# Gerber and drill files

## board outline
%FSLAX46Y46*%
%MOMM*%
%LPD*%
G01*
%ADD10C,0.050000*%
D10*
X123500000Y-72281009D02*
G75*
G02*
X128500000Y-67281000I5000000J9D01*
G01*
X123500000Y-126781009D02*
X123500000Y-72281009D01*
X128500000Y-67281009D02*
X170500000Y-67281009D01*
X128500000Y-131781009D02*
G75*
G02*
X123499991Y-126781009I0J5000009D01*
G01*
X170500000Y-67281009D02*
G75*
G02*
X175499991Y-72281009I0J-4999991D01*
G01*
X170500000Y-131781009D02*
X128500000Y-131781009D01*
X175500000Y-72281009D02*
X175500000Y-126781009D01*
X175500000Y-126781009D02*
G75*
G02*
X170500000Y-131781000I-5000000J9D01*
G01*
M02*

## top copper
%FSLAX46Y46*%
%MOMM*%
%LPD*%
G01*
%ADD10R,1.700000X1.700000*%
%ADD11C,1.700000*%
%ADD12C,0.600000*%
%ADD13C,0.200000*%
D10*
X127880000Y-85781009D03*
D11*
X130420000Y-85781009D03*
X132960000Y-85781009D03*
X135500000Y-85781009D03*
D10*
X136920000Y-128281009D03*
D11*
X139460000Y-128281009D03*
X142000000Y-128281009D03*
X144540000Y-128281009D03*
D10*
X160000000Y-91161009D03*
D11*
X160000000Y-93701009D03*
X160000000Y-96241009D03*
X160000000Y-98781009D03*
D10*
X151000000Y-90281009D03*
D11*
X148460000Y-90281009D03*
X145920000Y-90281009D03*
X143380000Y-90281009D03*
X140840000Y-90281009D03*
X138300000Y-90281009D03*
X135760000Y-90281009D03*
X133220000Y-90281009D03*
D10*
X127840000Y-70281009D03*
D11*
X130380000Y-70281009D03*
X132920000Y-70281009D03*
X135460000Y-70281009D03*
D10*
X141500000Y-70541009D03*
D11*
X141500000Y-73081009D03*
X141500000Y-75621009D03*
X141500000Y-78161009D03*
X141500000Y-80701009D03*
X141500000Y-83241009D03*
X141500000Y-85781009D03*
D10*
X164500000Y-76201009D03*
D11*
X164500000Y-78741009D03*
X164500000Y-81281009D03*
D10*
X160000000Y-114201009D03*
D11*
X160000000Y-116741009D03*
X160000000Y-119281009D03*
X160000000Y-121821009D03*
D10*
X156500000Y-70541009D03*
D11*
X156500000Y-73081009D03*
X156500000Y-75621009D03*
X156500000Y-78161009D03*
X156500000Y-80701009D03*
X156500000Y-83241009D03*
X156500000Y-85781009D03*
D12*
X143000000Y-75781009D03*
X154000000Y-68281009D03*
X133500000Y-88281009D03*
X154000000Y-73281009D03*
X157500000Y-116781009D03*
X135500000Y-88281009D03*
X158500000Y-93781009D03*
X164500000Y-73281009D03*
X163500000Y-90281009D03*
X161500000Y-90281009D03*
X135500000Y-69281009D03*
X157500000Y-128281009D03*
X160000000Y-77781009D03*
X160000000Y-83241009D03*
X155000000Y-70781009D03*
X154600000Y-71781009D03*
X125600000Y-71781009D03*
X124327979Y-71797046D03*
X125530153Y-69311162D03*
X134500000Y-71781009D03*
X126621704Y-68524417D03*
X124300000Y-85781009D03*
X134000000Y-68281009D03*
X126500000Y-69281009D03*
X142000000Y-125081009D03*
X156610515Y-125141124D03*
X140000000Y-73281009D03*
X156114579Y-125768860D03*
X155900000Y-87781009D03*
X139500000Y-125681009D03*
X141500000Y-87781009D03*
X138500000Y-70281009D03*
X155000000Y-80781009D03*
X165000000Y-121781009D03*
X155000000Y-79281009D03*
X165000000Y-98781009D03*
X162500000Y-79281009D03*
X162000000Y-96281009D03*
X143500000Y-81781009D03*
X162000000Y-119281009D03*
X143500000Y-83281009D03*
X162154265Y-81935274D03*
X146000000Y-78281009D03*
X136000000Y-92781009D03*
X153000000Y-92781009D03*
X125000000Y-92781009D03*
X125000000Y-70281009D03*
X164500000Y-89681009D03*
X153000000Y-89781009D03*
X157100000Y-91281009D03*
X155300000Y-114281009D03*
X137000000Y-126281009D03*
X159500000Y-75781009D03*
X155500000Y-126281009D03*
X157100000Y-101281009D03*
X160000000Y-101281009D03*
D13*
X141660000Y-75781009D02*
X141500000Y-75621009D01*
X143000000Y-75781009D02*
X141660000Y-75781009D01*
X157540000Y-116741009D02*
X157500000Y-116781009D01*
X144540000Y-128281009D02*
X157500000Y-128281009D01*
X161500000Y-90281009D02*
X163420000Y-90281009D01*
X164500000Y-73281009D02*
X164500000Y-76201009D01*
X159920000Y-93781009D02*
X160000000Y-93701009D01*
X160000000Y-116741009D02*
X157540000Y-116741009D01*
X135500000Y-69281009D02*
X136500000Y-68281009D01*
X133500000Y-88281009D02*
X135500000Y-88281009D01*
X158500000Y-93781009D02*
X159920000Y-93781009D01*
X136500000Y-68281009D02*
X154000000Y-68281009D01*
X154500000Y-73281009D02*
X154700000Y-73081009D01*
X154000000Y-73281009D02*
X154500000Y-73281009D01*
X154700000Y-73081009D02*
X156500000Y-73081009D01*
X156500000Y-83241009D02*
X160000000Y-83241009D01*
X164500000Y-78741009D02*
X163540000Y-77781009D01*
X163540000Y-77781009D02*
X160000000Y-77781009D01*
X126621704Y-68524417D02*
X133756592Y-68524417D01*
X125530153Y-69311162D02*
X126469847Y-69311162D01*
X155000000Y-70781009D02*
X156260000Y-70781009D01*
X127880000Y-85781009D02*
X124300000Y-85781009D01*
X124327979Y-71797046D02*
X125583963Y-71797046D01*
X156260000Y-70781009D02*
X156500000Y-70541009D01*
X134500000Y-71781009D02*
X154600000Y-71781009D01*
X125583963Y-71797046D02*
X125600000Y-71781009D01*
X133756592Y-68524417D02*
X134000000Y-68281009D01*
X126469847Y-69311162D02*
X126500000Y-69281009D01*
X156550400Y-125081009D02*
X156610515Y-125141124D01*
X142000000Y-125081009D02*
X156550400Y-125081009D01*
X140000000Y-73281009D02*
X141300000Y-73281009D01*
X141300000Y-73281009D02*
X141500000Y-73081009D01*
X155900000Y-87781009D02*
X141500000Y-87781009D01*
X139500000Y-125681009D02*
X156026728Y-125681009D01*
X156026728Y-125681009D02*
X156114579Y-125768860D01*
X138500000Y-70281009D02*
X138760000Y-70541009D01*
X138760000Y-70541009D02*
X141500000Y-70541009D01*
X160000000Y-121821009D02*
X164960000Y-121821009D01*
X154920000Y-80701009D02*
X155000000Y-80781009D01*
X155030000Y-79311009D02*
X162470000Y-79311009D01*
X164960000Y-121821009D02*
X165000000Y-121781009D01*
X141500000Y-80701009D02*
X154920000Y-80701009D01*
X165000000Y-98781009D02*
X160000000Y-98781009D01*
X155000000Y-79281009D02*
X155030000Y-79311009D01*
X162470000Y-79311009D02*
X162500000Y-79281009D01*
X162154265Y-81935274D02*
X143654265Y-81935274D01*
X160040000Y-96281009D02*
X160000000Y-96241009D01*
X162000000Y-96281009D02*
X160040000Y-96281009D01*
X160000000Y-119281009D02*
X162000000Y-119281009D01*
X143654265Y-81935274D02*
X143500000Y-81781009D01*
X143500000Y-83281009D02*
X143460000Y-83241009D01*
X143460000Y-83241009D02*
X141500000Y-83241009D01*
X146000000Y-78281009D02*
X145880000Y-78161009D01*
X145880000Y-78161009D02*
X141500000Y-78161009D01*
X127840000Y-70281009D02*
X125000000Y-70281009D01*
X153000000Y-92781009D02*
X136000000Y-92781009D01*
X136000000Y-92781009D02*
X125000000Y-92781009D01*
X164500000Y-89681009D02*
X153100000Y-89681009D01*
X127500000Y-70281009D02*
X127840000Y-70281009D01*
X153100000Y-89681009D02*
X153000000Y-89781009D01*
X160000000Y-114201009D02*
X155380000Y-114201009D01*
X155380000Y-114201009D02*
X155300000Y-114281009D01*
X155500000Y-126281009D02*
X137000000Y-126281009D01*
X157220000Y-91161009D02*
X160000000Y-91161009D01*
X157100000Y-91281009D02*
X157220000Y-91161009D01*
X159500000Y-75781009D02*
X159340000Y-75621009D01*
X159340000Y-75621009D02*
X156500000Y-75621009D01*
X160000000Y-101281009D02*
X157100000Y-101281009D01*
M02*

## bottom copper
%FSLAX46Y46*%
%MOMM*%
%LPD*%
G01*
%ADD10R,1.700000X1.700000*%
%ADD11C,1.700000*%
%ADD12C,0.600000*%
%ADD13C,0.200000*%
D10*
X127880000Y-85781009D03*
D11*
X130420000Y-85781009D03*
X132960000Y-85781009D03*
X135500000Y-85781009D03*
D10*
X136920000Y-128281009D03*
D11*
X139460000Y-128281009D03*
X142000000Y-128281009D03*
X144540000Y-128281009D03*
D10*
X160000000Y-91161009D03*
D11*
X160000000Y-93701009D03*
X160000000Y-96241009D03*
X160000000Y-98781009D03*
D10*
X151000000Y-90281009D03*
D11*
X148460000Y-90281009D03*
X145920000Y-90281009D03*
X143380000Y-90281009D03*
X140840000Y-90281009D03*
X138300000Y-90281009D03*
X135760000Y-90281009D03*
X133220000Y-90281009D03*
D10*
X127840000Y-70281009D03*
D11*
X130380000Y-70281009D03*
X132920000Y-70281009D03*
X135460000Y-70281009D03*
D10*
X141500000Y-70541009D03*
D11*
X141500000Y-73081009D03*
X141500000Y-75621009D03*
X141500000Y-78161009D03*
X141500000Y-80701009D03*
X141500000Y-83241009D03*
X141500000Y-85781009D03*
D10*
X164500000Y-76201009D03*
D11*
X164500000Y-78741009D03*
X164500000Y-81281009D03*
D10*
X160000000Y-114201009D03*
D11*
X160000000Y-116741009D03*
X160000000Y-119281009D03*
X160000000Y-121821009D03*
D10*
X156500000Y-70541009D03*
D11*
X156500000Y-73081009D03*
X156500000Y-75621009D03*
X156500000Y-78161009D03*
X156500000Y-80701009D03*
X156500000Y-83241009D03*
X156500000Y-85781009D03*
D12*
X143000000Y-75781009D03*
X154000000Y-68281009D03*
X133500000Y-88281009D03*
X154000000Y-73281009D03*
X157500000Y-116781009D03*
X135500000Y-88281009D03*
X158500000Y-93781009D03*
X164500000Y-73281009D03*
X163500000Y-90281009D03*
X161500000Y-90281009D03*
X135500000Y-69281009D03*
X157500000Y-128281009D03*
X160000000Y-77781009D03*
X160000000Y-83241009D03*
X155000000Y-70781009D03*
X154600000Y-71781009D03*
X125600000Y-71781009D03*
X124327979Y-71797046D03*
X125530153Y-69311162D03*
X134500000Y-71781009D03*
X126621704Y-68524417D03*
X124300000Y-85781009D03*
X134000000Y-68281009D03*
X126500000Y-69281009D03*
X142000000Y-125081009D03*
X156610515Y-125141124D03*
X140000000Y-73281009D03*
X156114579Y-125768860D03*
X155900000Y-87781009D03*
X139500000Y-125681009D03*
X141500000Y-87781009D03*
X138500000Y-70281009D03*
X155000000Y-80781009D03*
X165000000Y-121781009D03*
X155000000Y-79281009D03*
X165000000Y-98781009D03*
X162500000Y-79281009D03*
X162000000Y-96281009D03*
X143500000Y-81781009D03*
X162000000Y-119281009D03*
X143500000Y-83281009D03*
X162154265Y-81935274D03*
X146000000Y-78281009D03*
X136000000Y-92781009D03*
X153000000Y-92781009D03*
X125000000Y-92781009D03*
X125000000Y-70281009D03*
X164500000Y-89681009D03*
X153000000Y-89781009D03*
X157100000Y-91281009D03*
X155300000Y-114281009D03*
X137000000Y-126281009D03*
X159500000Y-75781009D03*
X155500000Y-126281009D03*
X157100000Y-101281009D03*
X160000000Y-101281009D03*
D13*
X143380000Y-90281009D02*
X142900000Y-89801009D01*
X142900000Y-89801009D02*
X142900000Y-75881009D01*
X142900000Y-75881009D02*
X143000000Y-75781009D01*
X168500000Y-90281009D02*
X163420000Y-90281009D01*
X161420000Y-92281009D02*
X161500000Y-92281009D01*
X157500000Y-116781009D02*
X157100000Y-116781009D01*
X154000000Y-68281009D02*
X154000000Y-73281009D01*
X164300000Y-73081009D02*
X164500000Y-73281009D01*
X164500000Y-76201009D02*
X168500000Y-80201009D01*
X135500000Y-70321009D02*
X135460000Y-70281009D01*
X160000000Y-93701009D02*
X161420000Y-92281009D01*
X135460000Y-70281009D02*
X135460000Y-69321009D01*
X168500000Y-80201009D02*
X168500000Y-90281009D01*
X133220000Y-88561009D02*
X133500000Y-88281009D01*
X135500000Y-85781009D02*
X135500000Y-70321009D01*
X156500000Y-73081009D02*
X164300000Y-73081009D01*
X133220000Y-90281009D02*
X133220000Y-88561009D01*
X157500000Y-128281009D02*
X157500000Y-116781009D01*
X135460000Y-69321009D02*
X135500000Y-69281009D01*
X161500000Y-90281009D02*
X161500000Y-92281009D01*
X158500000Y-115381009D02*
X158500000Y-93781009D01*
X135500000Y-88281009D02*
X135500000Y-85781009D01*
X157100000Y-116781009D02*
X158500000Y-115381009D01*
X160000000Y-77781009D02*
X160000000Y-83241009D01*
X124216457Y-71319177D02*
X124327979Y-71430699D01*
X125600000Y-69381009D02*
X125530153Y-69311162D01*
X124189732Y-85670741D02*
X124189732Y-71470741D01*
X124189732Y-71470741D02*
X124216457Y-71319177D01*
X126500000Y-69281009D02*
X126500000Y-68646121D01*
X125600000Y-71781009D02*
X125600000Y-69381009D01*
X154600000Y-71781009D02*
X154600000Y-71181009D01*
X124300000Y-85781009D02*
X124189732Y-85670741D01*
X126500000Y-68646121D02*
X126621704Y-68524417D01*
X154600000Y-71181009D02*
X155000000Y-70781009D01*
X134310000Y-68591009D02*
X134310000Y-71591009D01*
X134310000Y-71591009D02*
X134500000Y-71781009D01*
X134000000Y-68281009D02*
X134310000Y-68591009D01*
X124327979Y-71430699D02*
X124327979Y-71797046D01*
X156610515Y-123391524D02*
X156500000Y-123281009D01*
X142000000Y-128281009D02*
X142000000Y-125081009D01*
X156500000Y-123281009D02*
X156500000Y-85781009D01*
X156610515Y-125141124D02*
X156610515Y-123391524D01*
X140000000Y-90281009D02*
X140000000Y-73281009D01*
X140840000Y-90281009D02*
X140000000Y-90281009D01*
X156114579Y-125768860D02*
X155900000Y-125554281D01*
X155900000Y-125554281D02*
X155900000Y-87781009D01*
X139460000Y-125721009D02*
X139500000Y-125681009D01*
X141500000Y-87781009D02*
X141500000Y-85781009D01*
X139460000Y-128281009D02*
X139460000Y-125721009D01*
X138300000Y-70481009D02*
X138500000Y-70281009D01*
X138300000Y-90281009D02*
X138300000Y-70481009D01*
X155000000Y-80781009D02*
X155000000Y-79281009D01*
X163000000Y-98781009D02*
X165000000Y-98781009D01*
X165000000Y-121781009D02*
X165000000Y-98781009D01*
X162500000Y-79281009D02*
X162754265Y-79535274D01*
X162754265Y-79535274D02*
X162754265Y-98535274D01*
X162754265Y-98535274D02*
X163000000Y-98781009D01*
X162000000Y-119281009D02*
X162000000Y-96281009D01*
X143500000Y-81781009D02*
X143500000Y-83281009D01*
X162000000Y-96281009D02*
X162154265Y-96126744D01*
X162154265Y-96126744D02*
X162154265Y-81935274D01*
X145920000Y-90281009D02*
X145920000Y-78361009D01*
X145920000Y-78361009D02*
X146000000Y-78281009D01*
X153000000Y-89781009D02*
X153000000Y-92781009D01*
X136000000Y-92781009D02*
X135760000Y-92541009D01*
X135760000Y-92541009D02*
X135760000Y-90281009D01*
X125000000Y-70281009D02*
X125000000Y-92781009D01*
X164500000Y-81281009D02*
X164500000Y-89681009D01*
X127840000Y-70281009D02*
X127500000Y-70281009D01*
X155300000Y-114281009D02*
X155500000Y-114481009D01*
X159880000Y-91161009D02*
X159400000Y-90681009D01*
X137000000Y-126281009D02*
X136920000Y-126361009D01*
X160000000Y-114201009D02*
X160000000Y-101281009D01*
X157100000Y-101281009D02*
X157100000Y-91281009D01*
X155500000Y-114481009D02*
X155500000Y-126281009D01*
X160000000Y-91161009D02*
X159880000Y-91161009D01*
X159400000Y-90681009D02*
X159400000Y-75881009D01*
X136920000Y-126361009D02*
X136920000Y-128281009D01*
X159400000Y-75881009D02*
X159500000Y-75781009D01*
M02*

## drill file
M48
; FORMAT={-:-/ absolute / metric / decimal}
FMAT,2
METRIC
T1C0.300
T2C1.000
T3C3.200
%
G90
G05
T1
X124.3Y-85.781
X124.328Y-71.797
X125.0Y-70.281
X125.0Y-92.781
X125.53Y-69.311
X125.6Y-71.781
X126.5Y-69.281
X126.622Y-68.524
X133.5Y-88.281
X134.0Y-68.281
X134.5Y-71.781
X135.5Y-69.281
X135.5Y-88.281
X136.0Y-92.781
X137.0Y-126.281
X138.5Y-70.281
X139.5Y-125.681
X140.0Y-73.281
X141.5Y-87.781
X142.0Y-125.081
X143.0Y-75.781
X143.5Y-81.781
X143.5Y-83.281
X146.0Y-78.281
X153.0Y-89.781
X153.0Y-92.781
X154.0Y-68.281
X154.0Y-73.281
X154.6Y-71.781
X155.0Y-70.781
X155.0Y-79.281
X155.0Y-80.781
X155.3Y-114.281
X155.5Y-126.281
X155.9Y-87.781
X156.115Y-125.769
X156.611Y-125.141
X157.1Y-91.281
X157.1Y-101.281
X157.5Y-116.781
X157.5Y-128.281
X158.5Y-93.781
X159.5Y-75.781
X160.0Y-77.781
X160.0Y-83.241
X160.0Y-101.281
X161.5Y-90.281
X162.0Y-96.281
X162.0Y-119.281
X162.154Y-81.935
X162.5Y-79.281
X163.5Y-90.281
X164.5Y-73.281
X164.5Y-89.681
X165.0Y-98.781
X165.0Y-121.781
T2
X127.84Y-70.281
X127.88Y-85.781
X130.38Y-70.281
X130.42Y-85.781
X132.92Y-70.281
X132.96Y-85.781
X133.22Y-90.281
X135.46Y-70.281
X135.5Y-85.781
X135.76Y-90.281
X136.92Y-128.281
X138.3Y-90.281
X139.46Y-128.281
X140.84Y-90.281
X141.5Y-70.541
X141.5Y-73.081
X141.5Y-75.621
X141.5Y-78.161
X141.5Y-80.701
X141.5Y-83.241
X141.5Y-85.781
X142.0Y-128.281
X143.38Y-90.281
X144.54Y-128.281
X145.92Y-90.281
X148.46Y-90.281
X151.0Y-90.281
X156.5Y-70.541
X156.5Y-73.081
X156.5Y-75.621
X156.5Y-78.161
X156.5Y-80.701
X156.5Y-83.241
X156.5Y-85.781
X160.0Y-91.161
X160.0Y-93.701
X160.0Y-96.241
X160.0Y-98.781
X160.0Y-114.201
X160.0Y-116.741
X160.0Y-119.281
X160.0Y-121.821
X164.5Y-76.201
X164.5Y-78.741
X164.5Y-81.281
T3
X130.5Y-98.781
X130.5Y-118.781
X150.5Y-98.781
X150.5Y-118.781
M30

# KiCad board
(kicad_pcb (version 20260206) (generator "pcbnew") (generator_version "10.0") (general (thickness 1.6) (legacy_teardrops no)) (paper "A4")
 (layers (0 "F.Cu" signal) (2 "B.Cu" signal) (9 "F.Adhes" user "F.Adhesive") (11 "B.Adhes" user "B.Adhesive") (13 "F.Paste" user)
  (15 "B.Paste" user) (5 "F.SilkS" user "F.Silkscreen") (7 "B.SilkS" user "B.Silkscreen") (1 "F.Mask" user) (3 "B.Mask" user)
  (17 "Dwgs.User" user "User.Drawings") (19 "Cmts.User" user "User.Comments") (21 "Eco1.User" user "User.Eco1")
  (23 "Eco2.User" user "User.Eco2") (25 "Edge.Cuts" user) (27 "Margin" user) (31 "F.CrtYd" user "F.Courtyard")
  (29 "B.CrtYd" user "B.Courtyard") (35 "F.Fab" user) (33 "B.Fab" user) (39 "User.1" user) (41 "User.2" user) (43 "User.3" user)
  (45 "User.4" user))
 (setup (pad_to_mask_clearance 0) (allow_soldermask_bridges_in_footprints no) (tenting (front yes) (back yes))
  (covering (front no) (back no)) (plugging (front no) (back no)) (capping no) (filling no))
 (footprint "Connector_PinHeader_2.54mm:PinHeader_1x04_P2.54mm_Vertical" (layer "F.Cu") (at 127.88 85.781009 90)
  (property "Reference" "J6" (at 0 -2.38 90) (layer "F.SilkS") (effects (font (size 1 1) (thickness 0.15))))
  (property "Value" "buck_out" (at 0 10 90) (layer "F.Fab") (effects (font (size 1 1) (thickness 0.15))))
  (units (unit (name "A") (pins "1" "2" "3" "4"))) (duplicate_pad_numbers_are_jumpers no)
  (pad "1" thru_hole rect (at 0 0 90) (size 1.7 1.7) (drill 1) (layers "*.Cu" "*.Mask") (remove_unused_layers no) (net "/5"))
  (pad "2" thru_hole circle (at 0 2.54 90) (size 1.7 1.7) (drill 1) (layers "*.Cu" "*.Mask") (remove_unused_layers no)
   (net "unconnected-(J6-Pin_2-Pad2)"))
  (pad "3" thru_hole circle (at 0 5.08 90) (size 1.7 1.7) (drill 1) (layers "*.Cu" "*.Mask") (remove_unused_layers no)
   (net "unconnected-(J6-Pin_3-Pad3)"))
  (pad "4" thru_hole circle (at 0 7.62 90) (size 1.7 1.7) (drill 1) (layers "*.Cu" "*.Mask") (remove_unused_layers no) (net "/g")))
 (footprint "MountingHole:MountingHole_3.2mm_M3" (layer "F.Cu") (at 150.5 98.781009)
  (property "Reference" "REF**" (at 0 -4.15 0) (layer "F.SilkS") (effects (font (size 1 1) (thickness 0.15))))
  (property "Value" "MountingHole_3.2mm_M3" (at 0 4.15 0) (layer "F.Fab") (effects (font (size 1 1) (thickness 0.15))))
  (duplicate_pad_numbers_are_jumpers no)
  (pad "" np_thru_hole circle (at 0 0) (size 3.2 3.2) (drill 3.2) (layers "*.Cu" "*.Mask")))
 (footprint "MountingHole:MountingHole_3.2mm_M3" (layer "F.Cu") (at 130.5 118.781009)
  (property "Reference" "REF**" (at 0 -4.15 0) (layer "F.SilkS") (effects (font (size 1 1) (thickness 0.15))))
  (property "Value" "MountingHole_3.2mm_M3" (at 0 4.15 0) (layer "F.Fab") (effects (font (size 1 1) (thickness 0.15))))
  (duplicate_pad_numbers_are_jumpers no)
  (pad "" np_thru_hole circle (at 0 0) (size 3.2 3.2) (drill 3.2) (layers "*.Cu" "*.Mask")))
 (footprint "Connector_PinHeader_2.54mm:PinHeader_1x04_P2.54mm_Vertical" (layer "F.Cu") (at 136.92 128.281009 90)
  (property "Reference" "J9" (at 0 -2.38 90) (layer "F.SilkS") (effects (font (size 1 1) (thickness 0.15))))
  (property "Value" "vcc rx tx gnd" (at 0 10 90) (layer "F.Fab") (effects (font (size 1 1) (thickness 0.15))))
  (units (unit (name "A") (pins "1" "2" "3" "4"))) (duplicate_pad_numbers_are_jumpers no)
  (pad "1" thru_hole rect (at 0 0 90) (size 1.7 1.7) (drill 1) (layers "*.Cu" "*.Mask") (remove_unused_layers no) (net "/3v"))
  (pad "2" thru_hole circle (at 0 2.54 90) (size 1.7 1.7) (drill 1) (layers "*.Cu" "*.Mask") (remove_unused_layers no) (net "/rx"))
  (pad "3" thru_hole circle (at 0 5.08 90) (size 1.7 1.7) (drill 1) (layers "*.Cu" "*.Mask") (remove_unused_layers no) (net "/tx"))
  (pad "4" thru_hole circle (at 0 7.62 90) (size 1.7 1.7) (drill 1) (layers "*.Cu" "*.Mask") (remove_unused_layers no) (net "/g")))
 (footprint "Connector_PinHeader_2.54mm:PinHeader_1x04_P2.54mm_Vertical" (layer "F.Cu") (at 160 91.161009)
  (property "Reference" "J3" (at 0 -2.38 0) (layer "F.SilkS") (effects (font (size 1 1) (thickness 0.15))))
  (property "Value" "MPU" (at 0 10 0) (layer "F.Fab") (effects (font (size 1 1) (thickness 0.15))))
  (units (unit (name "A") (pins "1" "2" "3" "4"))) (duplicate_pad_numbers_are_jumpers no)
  (pad "1" thru_hole rect (at 0 0) (size 1.7 1.7) (drill 1) (layers "*.Cu" "*.Mask") (remove_unused_layers no) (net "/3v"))
  (pad "2" thru_hole circle (at 0 2.54) (size 1.7 1.7) (drill 1) (layers "*.Cu" "*.Mask") (remove_unused_layers no) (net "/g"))
  (pad "3" thru_hole circle (at 0 5.08) (size 1.7 1.7) (drill 1) (layers "*.Cu" "*.Mask") (remove_unused_layers no) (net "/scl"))
  (pad "4" thru_hole circle (at 0 7.62) (size 1.7 1.7) (drill 1) (layers "*.Cu" "*.Mask") (remove_unused_layers no) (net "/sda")))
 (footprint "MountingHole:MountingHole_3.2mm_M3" (layer "F.Cu") (at 150.5 118.781009)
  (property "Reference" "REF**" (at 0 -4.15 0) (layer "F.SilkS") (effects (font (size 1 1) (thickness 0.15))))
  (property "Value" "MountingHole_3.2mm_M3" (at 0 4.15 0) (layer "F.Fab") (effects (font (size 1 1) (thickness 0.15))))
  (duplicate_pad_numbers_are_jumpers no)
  (pad "" np_thru_hole circle (at 0 0) (size 3.2 3.2) (drill 3.2) (layers "*.Cu" "*.Mask")))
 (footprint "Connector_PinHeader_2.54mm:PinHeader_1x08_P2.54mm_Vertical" (layer "F.Cu") (at 151 90.281009 -90)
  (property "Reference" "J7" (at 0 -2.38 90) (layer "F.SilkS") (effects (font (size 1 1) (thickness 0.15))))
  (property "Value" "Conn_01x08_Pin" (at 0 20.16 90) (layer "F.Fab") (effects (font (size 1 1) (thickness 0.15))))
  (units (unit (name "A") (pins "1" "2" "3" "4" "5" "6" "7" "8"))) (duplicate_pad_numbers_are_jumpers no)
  (pad "1" thru_hole rect (at 0 0 270) (size 1.7 1.7) (drill 1) (layers "*.Cu" "*.Mask") (remove_unused_layers no)
   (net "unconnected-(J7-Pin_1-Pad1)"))
  (pad "2" thru_hole circle (at 0 2.54 270) (size 1.7 1.7) (drill 1) (layers "*.Cu" "*.Mask") (remove_unused_layers no)
   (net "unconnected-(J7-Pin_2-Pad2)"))
  (pad "3" thru_hole circle (at 0 5.08 270) (size 1.7 1.7) (drill 1) (layers "*.Cu" "*.Mask") (remove_unused_layers no) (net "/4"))
  (pad "4" thru_hole circle (at 0 7.62 270) (size 1.7 1.7) (drill 1) (layers "*.Cu" "*.Mask") (remove_unused_layers no) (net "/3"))
  (pad "5" thru_hole circle (at 0 10.16 270) (size 1.7 1.7) (drill 1) (layers "*.Cu" "*.Mask") (remove_unused_layers no) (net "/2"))
  (pad "6" thru_hole circle (at 0 12.7 270) (size 1.7 1.7) (drill 1) (layers "*.Cu" "*.Mask") (remove_unused_layers no) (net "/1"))
  (pad "7" thru_hole circle (at 0 15.24 270) (size 1.7 1.7) (drill 1) (layers "*.Cu" "*.Mask") (remove_unused_layers no) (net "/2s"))
  (pad "8" thru_hole circle (at 0 17.78 270) (size 1.7 1.7) (drill 1) (layers "*.Cu" "*.Mask") (remove_unused_layers no) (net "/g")))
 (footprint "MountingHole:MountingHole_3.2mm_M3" (layer "F.Cu") (at 130.5 98.781009)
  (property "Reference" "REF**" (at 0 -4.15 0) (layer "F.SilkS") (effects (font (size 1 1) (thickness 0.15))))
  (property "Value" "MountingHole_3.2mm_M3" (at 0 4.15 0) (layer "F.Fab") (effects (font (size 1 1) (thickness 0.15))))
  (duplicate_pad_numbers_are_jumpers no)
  (pad "" np_thru_hole circle (at 0 0) (size 3.2 3.2) (drill 3.2) (layers "*.Cu" "*.Mask")))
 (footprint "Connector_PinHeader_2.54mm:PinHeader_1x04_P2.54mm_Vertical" (layer "F.Cu") (at 127.84 70.281009 90)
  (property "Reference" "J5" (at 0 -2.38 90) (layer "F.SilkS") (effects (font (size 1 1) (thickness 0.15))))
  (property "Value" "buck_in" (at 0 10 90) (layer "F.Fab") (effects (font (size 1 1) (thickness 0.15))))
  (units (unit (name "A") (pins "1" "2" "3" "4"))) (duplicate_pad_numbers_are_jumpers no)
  (pad "1" thru_hole rect (at 0 0 90) (size 1.7 1.7) (drill 1) (layers "*.Cu" "*.Mask") (remove_unused_layers no) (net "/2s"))
  (pad "2" thru_hole circle (at 0 2.54 90) (size 1.7 1.7) (drill 1) (layers "*.Cu" "*.Mask") (remove_unused_layers no)
   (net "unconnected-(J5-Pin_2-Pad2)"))
  (pad "3" thru_hole circle (at 0 5.08 90) (size 1.7 1.7) (drill 1) (layers "*.Cu" "*.Mask") (remove_unused_layers no)
   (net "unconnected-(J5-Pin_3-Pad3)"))
  (pad "4" thru_hole circle (at 0 7.62 90) (size 1.7 1.7) (drill 1) (layers "*.Cu" "*.Mask") (remove_unused_layers no) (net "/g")))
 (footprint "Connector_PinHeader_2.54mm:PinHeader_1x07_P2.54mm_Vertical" (layer "F.Cu") (at 141.5 70.541009)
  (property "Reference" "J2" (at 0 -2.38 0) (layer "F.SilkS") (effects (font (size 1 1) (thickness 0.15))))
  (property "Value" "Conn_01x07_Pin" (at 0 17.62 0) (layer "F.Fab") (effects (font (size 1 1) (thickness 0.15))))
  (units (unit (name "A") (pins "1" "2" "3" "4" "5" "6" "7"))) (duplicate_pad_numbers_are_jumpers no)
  (pad "1" thru_hole rect (at 0 0) (size 1.7 1.7) (drill 1) (layers "*.Cu" "*.Mask") (remove_unused_layers no) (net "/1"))
  (pad "2" thru_hole circle (at 0 2.54) (size 1.7 1.7) (drill 1) (layers "*.Cu" "*.Mask") (remove_unused_layers no) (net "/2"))
  (pad "3" thru_hole circle (at 0 5.08) (size 1.7 1.7) (drill 1) (layers "*.Cu" "*.Mask") (remove_unused_layers no) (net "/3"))
  (pad "4" thru_hole circle (at 0 7.62) (size 1.7 1.7) (drill 1) (layers "*.Cu" "*.Mask") (remove_unused_layers no) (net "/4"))
  (pad "5" thru_hole circle (at 0 10.16) (size 1.7 1.7) (drill 1) (layers "*.Cu" "*.Mask") (remove_unused_layers no) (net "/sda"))
  (pad "6" thru_hole circle (at 0 12.7) (size 1.7 1.7) (drill 1) (layers "*.Cu" "*.Mask") (remove_unused_layers no) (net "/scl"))
  (pad "7" thru_hole circle (at 0 15.24) (size 1.7 1.7) (drill 1) (layers "*.Cu" "*.Mask") (remove_unused_layers no) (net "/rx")))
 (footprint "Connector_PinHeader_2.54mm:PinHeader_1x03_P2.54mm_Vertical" (layer "F.Cu") (at 164.5 76.201009)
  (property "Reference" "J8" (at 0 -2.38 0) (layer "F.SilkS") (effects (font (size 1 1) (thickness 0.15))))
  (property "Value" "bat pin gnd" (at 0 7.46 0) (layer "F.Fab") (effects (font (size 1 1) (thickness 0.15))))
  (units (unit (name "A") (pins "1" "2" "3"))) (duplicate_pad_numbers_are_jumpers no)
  (pad "1" thru_hole rect (at 0 0) (size 1.7 1.7) (drill 1) (layers "*.Cu" "*.Mask") (remove_unused_layers no) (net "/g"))
  (pad "2" thru_hole circle (at 0 2.54) (size 1.7 1.7) (drill 1) (layers "*.Cu" "*.Mask") (remove_unused_layers no) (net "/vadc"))
  (pad "3" thru_hole circle (at 0 5.08) (size 1.7 1.7) (drill 1) (layers "*.Cu" "*.Mask") (remove_unused_layers no) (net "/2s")))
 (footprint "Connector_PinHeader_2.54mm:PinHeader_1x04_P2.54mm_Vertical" (layer "F.Cu") (at 160 114.201009)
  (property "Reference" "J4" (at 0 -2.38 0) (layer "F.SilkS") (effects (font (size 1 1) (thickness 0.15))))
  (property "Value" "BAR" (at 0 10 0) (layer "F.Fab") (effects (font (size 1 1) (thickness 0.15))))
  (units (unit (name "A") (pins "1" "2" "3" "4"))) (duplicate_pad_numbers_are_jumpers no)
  (pad "1" thru_hole rect (at 0 0) (size 1.7 1.7) (drill 1) (layers "*.Cu" "*.Mask") (remove_unused_layers no) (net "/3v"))
  (pad "2" thru_hole circle (at 0 2.54) (size 1.7 1.7) (drill 1) (layers "*.Cu" "*.Mask") (remove_unused_layers no) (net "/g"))
  (pad "3" thru_hole circle (at 0 5.08) (size 1.7 1.7) (drill 1) (layers "*.Cu" "*.Mask") (remove_unused_layers no) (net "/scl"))
  (pad "4" thru_hole circle (at 0 7.62) (size 1.7 1.7) (drill 1) (layers "*.Cu" "*.Mask") (remove_unused_layers no) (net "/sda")))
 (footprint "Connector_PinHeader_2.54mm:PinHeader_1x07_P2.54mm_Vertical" (layer "F.Cu") (at 156.5 70.541009)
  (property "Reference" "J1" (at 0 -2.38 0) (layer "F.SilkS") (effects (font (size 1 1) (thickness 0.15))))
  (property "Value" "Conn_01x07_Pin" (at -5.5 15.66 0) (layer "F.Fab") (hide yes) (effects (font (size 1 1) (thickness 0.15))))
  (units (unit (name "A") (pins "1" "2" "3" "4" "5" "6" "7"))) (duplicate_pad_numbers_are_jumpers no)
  (pad "1" thru_hole rect (at 0 0) (size 1.7 1.7) (drill 1) (layers "*.Cu" "*.Mask") (remove_unused_layers no) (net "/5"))
  (pad "2" thru_hole circle (at 0 2.54) (size 1.7 1.7) (drill 1) (layers "*.Cu" "*.Mask") (remove_unused_layers no) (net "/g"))
  (pad "3" thru_hole circle (at 0 5.08) (size 1.7 1.7) (drill 1) (layers "*.Cu" "*.Mask") (remove_unused_layers no) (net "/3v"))
  (pad "4" thru_hole circle (at 0 7.62) (size 1.7 1.7) (drill 1) (layers "*.Cu" "*.Mask") (remove_unused_layers no)
   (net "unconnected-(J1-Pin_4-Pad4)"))
  (pad "5" thru_hole circle (at 0 10.16) (size 1.7 1.7) (drill 1) (layers "*.Cu" "*.Mask") (remove_unused_layers no)
   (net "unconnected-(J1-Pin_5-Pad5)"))
  (pad "6" thru_hole circle (at 0 12.7) (size 1.7 1.7) (drill 1) (layers "*.Cu" "*.Mask") (remove_unused_layers no) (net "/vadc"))
  (pad "7" thru_hole circle (at 0 15.24) (size 1.7 1.7) (drill 1) (layers "*.Cu" "*.Mask") (remove_unused_layers no) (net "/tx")))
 (gr_arc (start 123.5 72.281009) (mid 124.964466 68.745475) (end 128.5 67.281009) (stroke (width 0.05) (type default)) (layer "Edge.Cuts"))
 (gr_line (start 123.5 126.781009) (end 123.5 72.281009) (stroke (width 0.05) (type default)) (layer "Edge.Cuts"))
 (gr_line (start 128.5 67.281009) (end 170.5 67.281009) (stroke (width 0.05) (type default)) (layer "Edge.Cuts"))
 (gr_arc (start 128.5 131.781009) (mid 124.964466 130.316543) (end 123.5 126.781009) (stroke (width 0.05) (type default))
  (layer "Edge.Cuts"))
 (gr_arc (start 170.5 67.281009) (mid 174.035534 68.745475) (end 175.5 72.281009) (stroke (width 0.05) (type default)) (layer "Edge.Cuts"))
 (gr_line (start 170.5 131.781009) (end 128.5 131.781009) (stroke (width 0.05) (type default)) (layer "Edge.Cuts"))
 (gr_line (start 175.5 72.281009) (end 175.5 126.781009) (stroke (width 0.05) (type default)) (layer "Edge.Cuts"))
 (gr_arc (start 175.5 126.781009) (mid 174.035534 130.316543) (end 170.5 131.781009) (stroke (width 0.05) (type default))
  (layer "Edge.Cuts"))
 (segment (start 141.66 75.781009) (end 141.5 75.621009) (width 0.2) (layer "F.Cu") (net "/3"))
 (segment (start 143 75.781009) (end 141.66 75.781009) (width 0.2) (layer "F.Cu") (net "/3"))
 (via (at 143 75.781009) (size 0.6) (drill 0.3) (layers "F.Cu" "B.Cu") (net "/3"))
 (segment (start 143.38 90.281009) (end 142.9 89.801009) (width 0.2) (layer "B.Cu") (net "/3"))
 (segment (start 142.9 89.801009) (end 142.9 75.881009) (width 0.2) (layer "B.Cu") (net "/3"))
 (segment (start 142.9 75.881009) (end 143 75.781009) (width 0.2) (layer "B.Cu") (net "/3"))
 (segment (start 157.54 116.741009) (end 157.5 116.781009) (width 0.2) (layer "F.Cu") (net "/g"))
 (segment (start 144.54 128.281009) (end 157.5 128.281009) (width 0.2) (layer "F.Cu") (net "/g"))
 (segment (start 161.5 90.281009) (end 163.42 90.281009) (width 0.2) (layer "F.Cu") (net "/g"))
 (segment (start 164.5 73.281009) (end 164.5 76.201009) (width 0.2) (layer "F.Cu") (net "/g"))
 (segment (start 159.92 93.781009) (end 160 93.701009) (width 0.2) (layer "F.Cu") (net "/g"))
 (segment (start 160 116.741009) (end 157.54 116.741009) (width 0.2) (layer "F.Cu") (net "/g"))
 (segment (start 135.5 69.281009) (end 136.5 68.281009) (width 0.2) (layer "F.Cu") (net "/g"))
 (segment (start 133.5 88.281009) (end 135.5 88.281009) (width 0.2) (layer "F.Cu") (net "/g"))
 (segment (start 158.5 93.781009) (end 159.92 93.781009) (width 0.2) (layer "F.Cu") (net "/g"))
 (segment (start 136.5 68.281009) (end 154 68.281009) (width 0.2) (layer "F.Cu") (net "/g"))
 (segment (start 154.5 73.281009) (end 154.7 73.081009) (width 0.2) (layer "F.Cu") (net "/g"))
 (segment (start 154 73.281009) (end 154.5 73.281009) (width 0.2) (layer "F.Cu") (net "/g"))
 (segment (start 154.7 73.081009) (end 156.5 73.081009) (width 0.2) (layer "F.Cu") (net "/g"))
 (via (at 154 68.281009) (size 0.6) (drill 0.3) (layers "F.Cu" "B.Cu") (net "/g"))
 (via (at 133.5 88.281009) (size 0.6) (drill 0.3) (layers "F.Cu" "B.Cu") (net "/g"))
 (via (at 154 73.281009) (size 0.6) (drill 0.3) (layers "F.Cu" "B.Cu") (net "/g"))
 (via (at 157.5 116.781009) (size 0.6) (drill 0.3) (layers "F.Cu" "B.Cu") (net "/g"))
 (via (at 135.5 88.281009) (size 0.6) (drill 0.3) (layers "F.Cu" "B.Cu") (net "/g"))
 (via (at 158.5 93.781009) (size 0.6) (drill 0.3) (layers "F.Cu" "B.Cu") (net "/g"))
 (via (at 164.5 73.281009) (size 0.6) (drill 0.3) (layers "F.Cu" "B.Cu") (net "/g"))
 (via (at 163.5 90.281009) (size 0.6) (drill 0.3) (layers "F.Cu" "B.Cu") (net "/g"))
 (via (at 161.5 90.281009) (size 0.6) (drill 0.3) (layers "F.Cu" "B.Cu") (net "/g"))
 (via (at 135.5 69.281009) (size 0.6) (drill 0.3) (layers "F.Cu" "B.Cu") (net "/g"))
 (via (at 157.5 128.281009) (size 0.6) (drill 0.3) (layers "F.Cu" "B.Cu") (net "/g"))
 (segment (start 168.5 90.281009) (end 163.42 90.281009) (width 0.2) (layer "B.Cu") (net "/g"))
 (segment (start 161.42 92.281009) (end 161.5 92.281009) (width 0.2) (layer "B.Cu") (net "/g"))
 (segment (start 157.5 116.781009) (end 157.1 116.781009) (width 0.2) (layer "B.Cu") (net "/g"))
 (segment (start 154 68.281009) (end 154 73.281009) (width 0.2) (layer "B.Cu") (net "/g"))
 (segment (start 164.3 73.081009) (end 164.5 73.281009) (width 0.2) (layer "B.Cu") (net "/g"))
 (segment (start 164.5 76.201009) (end 168.5 80.201009) (width 0.2) (layer "B.Cu") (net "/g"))
 (segment (start 135.5 70.321009) (end 135.46 70.281009) (width 0.2) (layer "B.Cu") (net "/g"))
 (segment (start 160 93.701009) (end 161.42 92.281009) (width 0.2) (layer "B.Cu") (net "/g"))
 (segment (start 135.46 70.281009) (end 135.46 69.321009) (width 0.2) (layer "B.Cu") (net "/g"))
 (segment (start 168.5 80.201009) (end 168.5 90.281009) (width 0.2) (layer "B.Cu") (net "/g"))
 (segment (start 133.22 88.561009) (end 133.5 88.281009) (width 0.2) (layer "B.Cu") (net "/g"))
 (segment (start 135.5 85.781009) (end 135.5 70.321009) (width 0.2) (layer "B.Cu") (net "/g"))
 (segment (start 156.5 73.081009) (end 164.3 73.081009) (width 0.2) (layer "B.Cu") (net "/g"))
 (segment (start 133.22 90.281009) (end 133.22 88.561009) (width 0.2) (layer "B.Cu") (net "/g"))
 (segment (start 157.5 128.281009) (end 157.5 116.781009) (width 0.2) (layer "B.Cu") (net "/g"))
 (segment (start 135.46 69.321009) (end 135.5 69.281009) (width 0.2) (layer "B.Cu") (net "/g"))
 (segment (start 161.5 90.281009) (end 161.5 92.281009) (width 0.2) (layer "B.Cu") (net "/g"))
 (segment (start 158.5 115.381009) (end 158.5 93.781009) (width 0.2) (layer "B.Cu") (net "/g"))
 (segment (start 135.5 88.281009) (end 135.5 85.781009) (width 0.2) (layer "B.Cu") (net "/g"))
 (segment (start 157.1 116.781009) (end 158.5 115.381009) (width 0.2) (layer "B.Cu") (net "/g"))
 (segment (start 156.5 83.241009) (end 160 83.241009) (width 0.2) (layer "F.Cu") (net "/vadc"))
 (segment (start 164.5 78.741009) (end 163.54 77.781009) (width 0.2) (layer "F.Cu") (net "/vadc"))
 (segment (start 163.54 77.781009) (end 160 77.781009) (width 0.2) (layer "F.Cu") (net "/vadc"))
 (via (at 160 77.781009) (size 0.6) (drill 0.3) (layers "F.Cu" "B.Cu") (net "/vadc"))
 (via (at 160 83.241009) (size 0.6) (drill 0.3) (layers "F.Cu" "B.Cu") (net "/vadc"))
 (segment (start 160 77.781009) (end 160 83.241009) (width 0.2) (layer "B.Cu") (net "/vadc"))
 (segment (start 126.621704 68.524417) (end 133.756592 68.524417) (width 0.2) (layer "F.Cu") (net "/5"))
 (segment (start 125.530153 69.311162) (end 126.469847 69.311162) (width 0.2) (layer "F.Cu") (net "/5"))
 (segment (start 155 70.781009) (end 156.26 70.781009) (width 0.2) (layer "F.Cu") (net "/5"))
 (segment (start 127.88 85.781009) (end 124.3 85.781009) (width 0.2) (layer "F.Cu") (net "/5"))
 (segment (start 124.327979 71.797046) (end 125.583963 71.797046) (width 0.2) (layer "F.Cu") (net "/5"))
 (segment (start 156.26 70.781009) (end 156.5 70.541009) (width 0.2) (layer "F.Cu") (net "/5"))
 (segment (start 134.5 71.781009) (end 154.6 71.781009) (width 0.2) (layer "F.Cu") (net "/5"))
 (segment (start 125.583963 71.797046) (end 125.6 71.781009) (width 0.2) (layer "F.Cu") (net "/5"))
 (segment (start 133.756592 68.524417) (end 134 68.281009) (width 0.2) (layer "F.Cu") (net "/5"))
 (segment (start 126.469847 69.311162) (end 126.5 69.281009) (width 0.2) (layer "F.Cu") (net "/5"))
 (via (at 155 70.781009) (size 0.6) (drill 0.3) (layers "F.Cu" "B.Cu") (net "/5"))
 (via (at 154.6 71.781009) (size 0.6) (drill 0.3) (layers "F.Cu" "B.Cu") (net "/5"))
 (via (at 125.6 71.781009) (size 0.6) (drill 0.3) (layers "F.Cu" "B.Cu") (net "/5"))
 (via (at 124.327979 71.797046) (size 0.6) (drill 0.3) (layers "F.Cu" "B.Cu") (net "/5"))
 (via (at 125.530153 69.311162) (size 0.6) (drill 0.3) (layers "F.Cu" "B.Cu") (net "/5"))
 (via (at 134.5 71.781009) (size 0.6) (drill 0.3) (layers "F.Cu" "B.Cu") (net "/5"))
 (via (at 126.621704 68.524417) (size 0.6) (drill 0.3) (layers "F.Cu" "B.Cu") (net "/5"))
 (via (at 124.3 85.781009) (size 0.6) (drill 0.3) (layers "F.Cu" "B.Cu") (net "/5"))
 (via (at 134 68.281009) (size 0.6) (drill 0.3) (layers "F.Cu" "B.Cu") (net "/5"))
 (via (at 126.5 69.281009) (size 0.6) (drill 0.3) (layers "F.Cu" "B.Cu") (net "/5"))
 (segment (start 124.216457 71.319177) (end 124.327979 71.430699) (width 0.2) (layer "B.Cu") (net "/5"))
 (segment (start 125.6 69.381009) (end 125.530153 69.311162) (width 0.2) (layer "B.Cu") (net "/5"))
 (segment (start 124.189732 85.670741) (end 124.189732 71.470741) (width 0.2) (layer "B.Cu") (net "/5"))
 (segment (start 124.189732 71.470741) (end 124.216457 71.319177) (width 0.2) (layer "B.Cu") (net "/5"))
 (segment (start 126.5 69.281009) (end 126.5 68.646121) (width 0.2) (layer "B.Cu") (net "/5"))
 (segment (start 125.6 71.781009) (end 125.6 69.381009) (width 0.2) (layer "B.Cu") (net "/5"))
 (segment (start 154.6 71.781009) (end 154.6 71.181009) (width 0.2) (layer "B.Cu") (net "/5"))
 (segment (start 124.3 85.781009) (end 124.189732 85.670741) (width 0.2) (layer "B.Cu") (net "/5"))
 (segment (start 126.5 68.646121) (end 126.621704 68.524417) (width 0.2) (layer "B.Cu") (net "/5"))
 (segment (start 154.6 71.181009) (end 155 70.781009) (width 0.2) (layer "B.Cu") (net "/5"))
 (segment (start 134.31 68.591009) (end 134.31 71.591009) (width 0.2) (layer "B.Cu") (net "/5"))
 (segment (start 134.31 71.591009) (end 134.5 71.781009) (width 0.2) (layer "B.Cu") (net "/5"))
 (segment (start 134 68.281009) (end 134.31 68.591009) (width 0.2) (layer "B.Cu") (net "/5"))
 (segment (start 124.327979 71.430699) (end 124.327979 71.797046) (width 0.2) (layer "B.Cu") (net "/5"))
 (segment (start 156.5504 125.081009) (end 156.610515 125.141124) (width 0.2) (layer "F.Cu") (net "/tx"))
 (segment (start 142 125.081009) (end 156.5504 125.081009) (width 0.2) (layer "F.Cu") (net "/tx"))
 (via (at 142 125.081009) (size 0.6) (drill 0.3) (layers "F.Cu" "B.Cu") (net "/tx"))
 (via (at 156.610515 125.141124) (size 0.6) (drill 0.3) (layers "F.Cu" "B.Cu") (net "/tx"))
 (segment (start 156.610515 123.391524) (end 156.5 123.281009) (width 0.2) (layer "B.Cu") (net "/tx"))
 (segment (start 142 128.281009) (end 142 125.081009) (width 0.2) (layer "B.Cu") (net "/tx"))
 (segment (start 156.5 123.281009) (end 156.5 85.781009) (width 0.2) (layer "B.Cu") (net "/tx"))
 (segment (start 156.610515 125.141124) (end 156.610515 123.391524) (width 0.2) (layer "B.Cu") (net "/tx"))
 (segment (start 140 73.281009) (end 141.3 73.281009) (width 0.2) (layer "F.Cu") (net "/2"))
 (segment (start 141.3 73.281009) (end 141.5 73.081009) (width 0.2) (layer "F.Cu") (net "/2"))
 (via (at 140 73.281009) (size 0.6) (drill 0.3) (layers "F.Cu" "B.Cu") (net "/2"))
 (segment (start 140 90.281009) (end 140 73.281009) (width 0.2) (layer "B.Cu") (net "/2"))
 (segment (start 140.84 90.281009) (end 140 90.281009) (width 0.2) (layer "B.Cu") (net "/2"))
 (segment (start 155.9 87.781009) (end 141.5 87.781009) (width 0.2) (layer "F.Cu") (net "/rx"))
 (segment (start 139.5 125.681009) (end 156.026728 125.681009) (width 0.2) (layer "F.Cu") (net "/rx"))
 (segment (start 156.026728 125.681009) (end 156.114579 125.76886) (width 0.2) (layer "F.Cu") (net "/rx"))
 (via (at 156.114579 125.76886) (size 0.6) (drill 0.3) (layers "F.Cu" "B.Cu") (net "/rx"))
 (via (at 155.9 87.781009) (size 0.6) (drill 0.3) (layers "F.Cu" "B.Cu") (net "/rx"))
 (via (at 139.5 125.681009) (size 0.6) (drill 0.3) (layers "F.Cu" "B.Cu") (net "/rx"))
 (via (at 141.5 87.781009) (size 0.6) (drill 0.3) (layers "F.Cu" "B.Cu") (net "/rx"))
 (segment (start 156.114579 125.76886) (end 155.9 125.554281) (width 0.2) (layer "B.Cu") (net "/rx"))
 (segment (start 155.9 125.554281) (end 155.9 87.781009) (width 0.2) (layer "B.Cu") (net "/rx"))
 (segment (start 139.46 125.721009) (end 139.5 125.681009) (width 0.2) (layer "B.Cu") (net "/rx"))
 (segment (start 141.5 87.781009) (end 141.5 85.781009) (width 0.2) (layer "B.Cu") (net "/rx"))
 (segment (start 139.46 128.281009) (end 139.46 125.721009) (width 0.2) (layer "B.Cu") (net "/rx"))
 (segment (start 138.5 70.281009) (end 138.76 70.541009) (width 0.2) (layer "F.Cu") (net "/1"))
 (segment (start 138.76 70.541009) (end 141.5 70.541009) (width 0.2) (layer "F.Cu") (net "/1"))
 (via (at 138.5 70.281009) (size 0.6) (drill 0.3) (layers "F.Cu" "B.Cu") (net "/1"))
 (segment (start 138.3 70.481009) (end 138.5 70.281009) (width 0.2) (layer "B.Cu") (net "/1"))
 (segment (start 138.3 90.281009) (end 138.3 70.481009) (width 0.2) (layer "B.Cu") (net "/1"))
 (segment (start 160 121.821009) (end 164.96 121.821009) (width 0.2) (layer "F.Cu") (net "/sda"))
 (segment (start 154.92 80.701009) (end 155 80.781009) (width 0.2) (layer "F.Cu") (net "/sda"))
 (segment (start 155.03 79.311009) (end 162.47 79.311009) (width 0.2) (layer "F.Cu") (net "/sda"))
 (segment (start 164.96 121.821009) (end 165 121.781009) (width 0.2) (layer "F.Cu") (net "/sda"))
 (segment (start 141.5 80.701009) (end 154.92 80.701009) (width 0.2) (layer "F.Cu") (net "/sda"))
 (segment (start 165 98.781009) (end 160 98.781009) (width 0.2) (layer "F.Cu") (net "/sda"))
 (segment (start 155 79.281009) (end 155.03 79.311009) (width 0.2) (layer "F.Cu") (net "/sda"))
 (segment (start 162.47 79.311009) (end 162.5 79.281009) (width 0.2) (layer "F.Cu") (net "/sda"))
 (via (at 155 80.781009) (size 0.6) (drill 0.3) (layers "F.Cu" "B.Cu") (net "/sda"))
 (via (at 165 121.781009) (size 0.6) (drill 0.3) (layers "F.Cu" "B.Cu") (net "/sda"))
 (via (at 155 79.281009) (size 0.6) (drill 0.3) (layers "F.Cu" "B.Cu") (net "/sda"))
 (via (at 165 98.781009) (size 0.6) (drill 0.3) (layers "F.Cu" "B.Cu") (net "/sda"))
 (via (at 162.5 79.281009) (size 0.6) (drill 0.3) (layers "F.Cu" "B.Cu") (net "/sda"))
 (segment (start 155 80.781009) (end 155 79.281009) (width 0.2) (layer "B.Cu") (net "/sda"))
 (segment (start 163 98.781009) (end 165 98.781009) (width 0.2) (layer "B.Cu") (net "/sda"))
 (segment (start 165 121.781009) (end 165 98.781009) (width 0.2) (layer "B.Cu") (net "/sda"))
 (segment (start 162.5 79.281009) (end 162.754265 79.535274) (width 0.2) (layer "B.Cu") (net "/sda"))
 (segment (start 162.754265 79.535274) (end 162.754265 98.535274) (width 0.2) (layer "B.Cu") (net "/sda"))
 (segment (start 162.754265 98.535274) (end 163 98.781009) (width 0.2) (layer "B.Cu") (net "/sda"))
 (segment (start 162.154265 81.935274) (end 143.654265 81.935274) (width 0.2) (layer "F.Cu") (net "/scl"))
 (segment (start 160.04 96.281009) (end 160 96.241009) (width 0.2) (layer "F.Cu") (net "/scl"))
 (segment (start 162 96.281009) (end 160.04 96.281009) (width 0.2) (layer "F.Cu") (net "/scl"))
 (segment (start 160 119.281009) (end 162 119.281009) (width 0.2) (layer "F.Cu") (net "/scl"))
 (segment (start 143.654265 81.935274) (end 143.5 81.781009) (width 0.2) (layer "F.Cu") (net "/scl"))
 (segment (start 143.5 83.281009) (end 143.46 83.241009) (width 0.2) (layer "F.Cu") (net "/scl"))
 (segment (start 143.46 83.241009) (end 141.5 83.241009) (width 0.2) (layer "F.Cu") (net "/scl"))
 (via (at 162 96.281009) (size 0.6) (drill 0.3) (layers "F.Cu" "B.Cu") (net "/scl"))
 (via (at 143.5 81.781009) (size 0.6) (drill 0.3) (layers "F.Cu" "B.Cu") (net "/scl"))
 (via (at 162 119.281009) (size 0.6) (drill 0.3) (layers "F.Cu" "B.Cu") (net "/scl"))
 (via (at 143.5 83.281009) (size 0.6) (drill 0.3) (layers "F.Cu" "B.Cu") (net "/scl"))
 (via (at 162.154265 81.935274) (size 0.6) (drill 0.3) (layers "F.Cu" "B.Cu") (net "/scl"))
 (segment (start 162 119.281009) (end 162 96.281009) (width 0.2) (layer "B.Cu") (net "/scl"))
 (segment (start 143.5 81.781009) (end 143.5 83.281009) (width 0.2) (layer "B.Cu") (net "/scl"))
 (segment (start 162 96.281009) (end 162.154265 96.126744) (width 0.2) (layer "B.Cu") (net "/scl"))
 (segment (start 162.154265 96.126744) (end 162.154265 81.935274) (width 0.2) (layer "B.Cu") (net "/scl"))
 (segment (start 146 78.281009) (end 145.88 78.161009) (width 0.2) (layer "F.Cu") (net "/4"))
 (segment (start 145.88 78.161009) (end 141.5 78.161009) (width 0.2) (layer "F.Cu") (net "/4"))
 (via (at 146 78.281009) (size 0.6) (drill 0.3) (layers "F.Cu" "B.Cu") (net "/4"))
 (segment (start 145.92 90.281009) (end 145.92 78.361009) (width 0.2) (layer "B.Cu") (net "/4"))
 (segment (start 145.92 78.361009) (end 146 78.281009) (width 0.2) (layer "B.Cu") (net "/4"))
 (segment (start 127.84 70.281009) (end 125 70.281009) (width 0.2) (layer "F.Cu") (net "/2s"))
 (segment (start 153 92.781009) (end 136 92.781009) (width 0.2) (layer "F.Cu") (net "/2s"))
 (segment (start 136 92.781009) (end 125 92.781009) (width 0.2) (layer "F.Cu") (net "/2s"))
 (segment (start 164.5 89.681009) (end 153.1 89.681009) (width 0.2) (layer "F.Cu") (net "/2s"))
 (segment (start 127.5 70.281009) (end 127.84 70.281009) (width 0.2) (layer "F.Cu") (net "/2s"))
 (segment (start 153.1 89.681009) (end 153 89.781009) (width 0.2) (layer "F.Cu") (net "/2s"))
 (via (at 136 92.781009) (size 0.6) (drill 0.3) (layers "F.Cu" "B.Cu") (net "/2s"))
 (via (at 153 92.781009) (size 0.6) (drill 0.3) (layers "F.Cu" "B.Cu") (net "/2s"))
 (via (at 125 92.781009) (size 0.6) (drill 0.3) (layers "F.Cu" "B.Cu") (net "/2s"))
 (via (at 125 70.281009) (size 0.6) (drill 0.3) (layers "F.Cu" "B.Cu") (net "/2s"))
 (via (at 164.5 89.681009) (size 0.6) (drill 0.3) (layers "F.Cu" "B.Cu") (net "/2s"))
 (via (at 153 89.781009) (size 0.6) (drill 0.3) (layers "F.Cu" "B.Cu") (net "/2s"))
 (segment (start 153 89.781009) (end 153 92.781009) (width 0.2) (layer "B.Cu") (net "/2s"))
 (segment (start 136 92.781009) (end 135.76 92.541009) (width 0.2) (layer "B.Cu") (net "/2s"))
 (segment (start 135.76 92.541009) (end 135.76 90.281009) (width 0.2) (layer "B.Cu") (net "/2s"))
 (segment (start 125 70.281009) (end 125 92.781009) (width 0.2) (layer "B.Cu") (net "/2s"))
 (segment (start 164.5 81.281009) (end 164.5 89.681009) (width 0.2) (layer "B.Cu") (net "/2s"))
 (segment (start 127.84 70.281009) (end 127.5 70.281009) (width 0.2) (layer "B.Cu") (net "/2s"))
 (segment (start 160 114.201009) (end 155.38 114.201009) (width 0.2) (layer "F.Cu") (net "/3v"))
 (segment (start 155.38 114.201009) (end 155.3 114.281009) (width 0.2) (layer "F.Cu") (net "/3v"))
 (segment (start 155.5 126.281009) (end 137 126.281009) (width 0.2) (layer "F.Cu") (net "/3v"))
 (segment (start 157.22 91.161009) (end 160 91.161009) (width 0.2) (layer "F.Cu") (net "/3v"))
 (segment (start 157.1 91.281009) (end 157.22 91.161009) (width 0.2) (layer "F.Cu") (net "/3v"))
 (segment (start 159.5 75.781009) (end 159.34 75.621009) (width 0.2) (layer "F.Cu") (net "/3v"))
 (segment (start 159.34 75.621009) (end 156.5 75.621009) (width 0.2) (layer "F.Cu") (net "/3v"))
 (segment (start 160 101.281009) (end 157.1 101.281009) (width 0.2) (layer "F.Cu") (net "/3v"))
 (via (at 157.1 91.281009) (size 0.6) (drill 0.3) (layers "F.Cu" "B.Cu") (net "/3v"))
 (via (at 155.3 114.281009) (size 0.6) (drill 0.3) (layers "F.Cu" "B.Cu") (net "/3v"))
 (via (at 137 126.281009) (size 0.6) (drill 0.3) (layers "F.Cu" "B.Cu") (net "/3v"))
 (via (at 159.5 75.781009) (size 0.6) (drill 0.3) (layers "F.Cu" "B.Cu") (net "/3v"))
 (via (at 155.5 126.281009) (size 0.6) (drill 0.3) (layers "F.Cu" "B.Cu") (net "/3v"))
 (via (at 157.1 101.281009) (size 0.6) (drill 0.3) (layers "F.Cu" "B.Cu") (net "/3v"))
 (via (at 160 101.281009) (size 0.6) (drill 0.3) (layers "F.Cu" "B.Cu") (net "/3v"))
 (segment (start 155.3 114.281009) (end 155.5 114.481009) (width 0.2) (layer "B.Cu") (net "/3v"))
 (segment (start 159.88 91.161009) (end 159.4 90.681009) (width 0.2) (layer "B.Cu") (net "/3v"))
 (segment (start 137 126.281009) (end 136.92 126.361009) (width 0.2) (layer "B.Cu") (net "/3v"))
 (segment (start 160 114.201009) (end 160 101.281009) (width 0.2) (layer "B.Cu") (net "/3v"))
 (segment (start 157.1 101.281009) (end 157.1 91.281009) (width 0.2) (layer "B.Cu") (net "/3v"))
 (segment (start 155.5 114.481009) (end 155.5 126.281009) (width 0.2) (layer "B.Cu") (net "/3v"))
 (segment (start 160 91.161009) (end 159.88 91.161009) (width 0.2) (layer "B.Cu") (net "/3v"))
 (segment (start 159.4 90.681009) (end 159.4 75.881009) (width 0.2) (layer "B.Cu") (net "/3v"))
 (segment (start 136.92 126.361009) (end 136.92 128.281009) (width 0.2) (layer "B.Cu") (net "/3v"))
 (segment (start 159.4 75.881009) (end 159.5 75.781009) (width 0.2) (layer "B.Cu") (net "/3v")))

